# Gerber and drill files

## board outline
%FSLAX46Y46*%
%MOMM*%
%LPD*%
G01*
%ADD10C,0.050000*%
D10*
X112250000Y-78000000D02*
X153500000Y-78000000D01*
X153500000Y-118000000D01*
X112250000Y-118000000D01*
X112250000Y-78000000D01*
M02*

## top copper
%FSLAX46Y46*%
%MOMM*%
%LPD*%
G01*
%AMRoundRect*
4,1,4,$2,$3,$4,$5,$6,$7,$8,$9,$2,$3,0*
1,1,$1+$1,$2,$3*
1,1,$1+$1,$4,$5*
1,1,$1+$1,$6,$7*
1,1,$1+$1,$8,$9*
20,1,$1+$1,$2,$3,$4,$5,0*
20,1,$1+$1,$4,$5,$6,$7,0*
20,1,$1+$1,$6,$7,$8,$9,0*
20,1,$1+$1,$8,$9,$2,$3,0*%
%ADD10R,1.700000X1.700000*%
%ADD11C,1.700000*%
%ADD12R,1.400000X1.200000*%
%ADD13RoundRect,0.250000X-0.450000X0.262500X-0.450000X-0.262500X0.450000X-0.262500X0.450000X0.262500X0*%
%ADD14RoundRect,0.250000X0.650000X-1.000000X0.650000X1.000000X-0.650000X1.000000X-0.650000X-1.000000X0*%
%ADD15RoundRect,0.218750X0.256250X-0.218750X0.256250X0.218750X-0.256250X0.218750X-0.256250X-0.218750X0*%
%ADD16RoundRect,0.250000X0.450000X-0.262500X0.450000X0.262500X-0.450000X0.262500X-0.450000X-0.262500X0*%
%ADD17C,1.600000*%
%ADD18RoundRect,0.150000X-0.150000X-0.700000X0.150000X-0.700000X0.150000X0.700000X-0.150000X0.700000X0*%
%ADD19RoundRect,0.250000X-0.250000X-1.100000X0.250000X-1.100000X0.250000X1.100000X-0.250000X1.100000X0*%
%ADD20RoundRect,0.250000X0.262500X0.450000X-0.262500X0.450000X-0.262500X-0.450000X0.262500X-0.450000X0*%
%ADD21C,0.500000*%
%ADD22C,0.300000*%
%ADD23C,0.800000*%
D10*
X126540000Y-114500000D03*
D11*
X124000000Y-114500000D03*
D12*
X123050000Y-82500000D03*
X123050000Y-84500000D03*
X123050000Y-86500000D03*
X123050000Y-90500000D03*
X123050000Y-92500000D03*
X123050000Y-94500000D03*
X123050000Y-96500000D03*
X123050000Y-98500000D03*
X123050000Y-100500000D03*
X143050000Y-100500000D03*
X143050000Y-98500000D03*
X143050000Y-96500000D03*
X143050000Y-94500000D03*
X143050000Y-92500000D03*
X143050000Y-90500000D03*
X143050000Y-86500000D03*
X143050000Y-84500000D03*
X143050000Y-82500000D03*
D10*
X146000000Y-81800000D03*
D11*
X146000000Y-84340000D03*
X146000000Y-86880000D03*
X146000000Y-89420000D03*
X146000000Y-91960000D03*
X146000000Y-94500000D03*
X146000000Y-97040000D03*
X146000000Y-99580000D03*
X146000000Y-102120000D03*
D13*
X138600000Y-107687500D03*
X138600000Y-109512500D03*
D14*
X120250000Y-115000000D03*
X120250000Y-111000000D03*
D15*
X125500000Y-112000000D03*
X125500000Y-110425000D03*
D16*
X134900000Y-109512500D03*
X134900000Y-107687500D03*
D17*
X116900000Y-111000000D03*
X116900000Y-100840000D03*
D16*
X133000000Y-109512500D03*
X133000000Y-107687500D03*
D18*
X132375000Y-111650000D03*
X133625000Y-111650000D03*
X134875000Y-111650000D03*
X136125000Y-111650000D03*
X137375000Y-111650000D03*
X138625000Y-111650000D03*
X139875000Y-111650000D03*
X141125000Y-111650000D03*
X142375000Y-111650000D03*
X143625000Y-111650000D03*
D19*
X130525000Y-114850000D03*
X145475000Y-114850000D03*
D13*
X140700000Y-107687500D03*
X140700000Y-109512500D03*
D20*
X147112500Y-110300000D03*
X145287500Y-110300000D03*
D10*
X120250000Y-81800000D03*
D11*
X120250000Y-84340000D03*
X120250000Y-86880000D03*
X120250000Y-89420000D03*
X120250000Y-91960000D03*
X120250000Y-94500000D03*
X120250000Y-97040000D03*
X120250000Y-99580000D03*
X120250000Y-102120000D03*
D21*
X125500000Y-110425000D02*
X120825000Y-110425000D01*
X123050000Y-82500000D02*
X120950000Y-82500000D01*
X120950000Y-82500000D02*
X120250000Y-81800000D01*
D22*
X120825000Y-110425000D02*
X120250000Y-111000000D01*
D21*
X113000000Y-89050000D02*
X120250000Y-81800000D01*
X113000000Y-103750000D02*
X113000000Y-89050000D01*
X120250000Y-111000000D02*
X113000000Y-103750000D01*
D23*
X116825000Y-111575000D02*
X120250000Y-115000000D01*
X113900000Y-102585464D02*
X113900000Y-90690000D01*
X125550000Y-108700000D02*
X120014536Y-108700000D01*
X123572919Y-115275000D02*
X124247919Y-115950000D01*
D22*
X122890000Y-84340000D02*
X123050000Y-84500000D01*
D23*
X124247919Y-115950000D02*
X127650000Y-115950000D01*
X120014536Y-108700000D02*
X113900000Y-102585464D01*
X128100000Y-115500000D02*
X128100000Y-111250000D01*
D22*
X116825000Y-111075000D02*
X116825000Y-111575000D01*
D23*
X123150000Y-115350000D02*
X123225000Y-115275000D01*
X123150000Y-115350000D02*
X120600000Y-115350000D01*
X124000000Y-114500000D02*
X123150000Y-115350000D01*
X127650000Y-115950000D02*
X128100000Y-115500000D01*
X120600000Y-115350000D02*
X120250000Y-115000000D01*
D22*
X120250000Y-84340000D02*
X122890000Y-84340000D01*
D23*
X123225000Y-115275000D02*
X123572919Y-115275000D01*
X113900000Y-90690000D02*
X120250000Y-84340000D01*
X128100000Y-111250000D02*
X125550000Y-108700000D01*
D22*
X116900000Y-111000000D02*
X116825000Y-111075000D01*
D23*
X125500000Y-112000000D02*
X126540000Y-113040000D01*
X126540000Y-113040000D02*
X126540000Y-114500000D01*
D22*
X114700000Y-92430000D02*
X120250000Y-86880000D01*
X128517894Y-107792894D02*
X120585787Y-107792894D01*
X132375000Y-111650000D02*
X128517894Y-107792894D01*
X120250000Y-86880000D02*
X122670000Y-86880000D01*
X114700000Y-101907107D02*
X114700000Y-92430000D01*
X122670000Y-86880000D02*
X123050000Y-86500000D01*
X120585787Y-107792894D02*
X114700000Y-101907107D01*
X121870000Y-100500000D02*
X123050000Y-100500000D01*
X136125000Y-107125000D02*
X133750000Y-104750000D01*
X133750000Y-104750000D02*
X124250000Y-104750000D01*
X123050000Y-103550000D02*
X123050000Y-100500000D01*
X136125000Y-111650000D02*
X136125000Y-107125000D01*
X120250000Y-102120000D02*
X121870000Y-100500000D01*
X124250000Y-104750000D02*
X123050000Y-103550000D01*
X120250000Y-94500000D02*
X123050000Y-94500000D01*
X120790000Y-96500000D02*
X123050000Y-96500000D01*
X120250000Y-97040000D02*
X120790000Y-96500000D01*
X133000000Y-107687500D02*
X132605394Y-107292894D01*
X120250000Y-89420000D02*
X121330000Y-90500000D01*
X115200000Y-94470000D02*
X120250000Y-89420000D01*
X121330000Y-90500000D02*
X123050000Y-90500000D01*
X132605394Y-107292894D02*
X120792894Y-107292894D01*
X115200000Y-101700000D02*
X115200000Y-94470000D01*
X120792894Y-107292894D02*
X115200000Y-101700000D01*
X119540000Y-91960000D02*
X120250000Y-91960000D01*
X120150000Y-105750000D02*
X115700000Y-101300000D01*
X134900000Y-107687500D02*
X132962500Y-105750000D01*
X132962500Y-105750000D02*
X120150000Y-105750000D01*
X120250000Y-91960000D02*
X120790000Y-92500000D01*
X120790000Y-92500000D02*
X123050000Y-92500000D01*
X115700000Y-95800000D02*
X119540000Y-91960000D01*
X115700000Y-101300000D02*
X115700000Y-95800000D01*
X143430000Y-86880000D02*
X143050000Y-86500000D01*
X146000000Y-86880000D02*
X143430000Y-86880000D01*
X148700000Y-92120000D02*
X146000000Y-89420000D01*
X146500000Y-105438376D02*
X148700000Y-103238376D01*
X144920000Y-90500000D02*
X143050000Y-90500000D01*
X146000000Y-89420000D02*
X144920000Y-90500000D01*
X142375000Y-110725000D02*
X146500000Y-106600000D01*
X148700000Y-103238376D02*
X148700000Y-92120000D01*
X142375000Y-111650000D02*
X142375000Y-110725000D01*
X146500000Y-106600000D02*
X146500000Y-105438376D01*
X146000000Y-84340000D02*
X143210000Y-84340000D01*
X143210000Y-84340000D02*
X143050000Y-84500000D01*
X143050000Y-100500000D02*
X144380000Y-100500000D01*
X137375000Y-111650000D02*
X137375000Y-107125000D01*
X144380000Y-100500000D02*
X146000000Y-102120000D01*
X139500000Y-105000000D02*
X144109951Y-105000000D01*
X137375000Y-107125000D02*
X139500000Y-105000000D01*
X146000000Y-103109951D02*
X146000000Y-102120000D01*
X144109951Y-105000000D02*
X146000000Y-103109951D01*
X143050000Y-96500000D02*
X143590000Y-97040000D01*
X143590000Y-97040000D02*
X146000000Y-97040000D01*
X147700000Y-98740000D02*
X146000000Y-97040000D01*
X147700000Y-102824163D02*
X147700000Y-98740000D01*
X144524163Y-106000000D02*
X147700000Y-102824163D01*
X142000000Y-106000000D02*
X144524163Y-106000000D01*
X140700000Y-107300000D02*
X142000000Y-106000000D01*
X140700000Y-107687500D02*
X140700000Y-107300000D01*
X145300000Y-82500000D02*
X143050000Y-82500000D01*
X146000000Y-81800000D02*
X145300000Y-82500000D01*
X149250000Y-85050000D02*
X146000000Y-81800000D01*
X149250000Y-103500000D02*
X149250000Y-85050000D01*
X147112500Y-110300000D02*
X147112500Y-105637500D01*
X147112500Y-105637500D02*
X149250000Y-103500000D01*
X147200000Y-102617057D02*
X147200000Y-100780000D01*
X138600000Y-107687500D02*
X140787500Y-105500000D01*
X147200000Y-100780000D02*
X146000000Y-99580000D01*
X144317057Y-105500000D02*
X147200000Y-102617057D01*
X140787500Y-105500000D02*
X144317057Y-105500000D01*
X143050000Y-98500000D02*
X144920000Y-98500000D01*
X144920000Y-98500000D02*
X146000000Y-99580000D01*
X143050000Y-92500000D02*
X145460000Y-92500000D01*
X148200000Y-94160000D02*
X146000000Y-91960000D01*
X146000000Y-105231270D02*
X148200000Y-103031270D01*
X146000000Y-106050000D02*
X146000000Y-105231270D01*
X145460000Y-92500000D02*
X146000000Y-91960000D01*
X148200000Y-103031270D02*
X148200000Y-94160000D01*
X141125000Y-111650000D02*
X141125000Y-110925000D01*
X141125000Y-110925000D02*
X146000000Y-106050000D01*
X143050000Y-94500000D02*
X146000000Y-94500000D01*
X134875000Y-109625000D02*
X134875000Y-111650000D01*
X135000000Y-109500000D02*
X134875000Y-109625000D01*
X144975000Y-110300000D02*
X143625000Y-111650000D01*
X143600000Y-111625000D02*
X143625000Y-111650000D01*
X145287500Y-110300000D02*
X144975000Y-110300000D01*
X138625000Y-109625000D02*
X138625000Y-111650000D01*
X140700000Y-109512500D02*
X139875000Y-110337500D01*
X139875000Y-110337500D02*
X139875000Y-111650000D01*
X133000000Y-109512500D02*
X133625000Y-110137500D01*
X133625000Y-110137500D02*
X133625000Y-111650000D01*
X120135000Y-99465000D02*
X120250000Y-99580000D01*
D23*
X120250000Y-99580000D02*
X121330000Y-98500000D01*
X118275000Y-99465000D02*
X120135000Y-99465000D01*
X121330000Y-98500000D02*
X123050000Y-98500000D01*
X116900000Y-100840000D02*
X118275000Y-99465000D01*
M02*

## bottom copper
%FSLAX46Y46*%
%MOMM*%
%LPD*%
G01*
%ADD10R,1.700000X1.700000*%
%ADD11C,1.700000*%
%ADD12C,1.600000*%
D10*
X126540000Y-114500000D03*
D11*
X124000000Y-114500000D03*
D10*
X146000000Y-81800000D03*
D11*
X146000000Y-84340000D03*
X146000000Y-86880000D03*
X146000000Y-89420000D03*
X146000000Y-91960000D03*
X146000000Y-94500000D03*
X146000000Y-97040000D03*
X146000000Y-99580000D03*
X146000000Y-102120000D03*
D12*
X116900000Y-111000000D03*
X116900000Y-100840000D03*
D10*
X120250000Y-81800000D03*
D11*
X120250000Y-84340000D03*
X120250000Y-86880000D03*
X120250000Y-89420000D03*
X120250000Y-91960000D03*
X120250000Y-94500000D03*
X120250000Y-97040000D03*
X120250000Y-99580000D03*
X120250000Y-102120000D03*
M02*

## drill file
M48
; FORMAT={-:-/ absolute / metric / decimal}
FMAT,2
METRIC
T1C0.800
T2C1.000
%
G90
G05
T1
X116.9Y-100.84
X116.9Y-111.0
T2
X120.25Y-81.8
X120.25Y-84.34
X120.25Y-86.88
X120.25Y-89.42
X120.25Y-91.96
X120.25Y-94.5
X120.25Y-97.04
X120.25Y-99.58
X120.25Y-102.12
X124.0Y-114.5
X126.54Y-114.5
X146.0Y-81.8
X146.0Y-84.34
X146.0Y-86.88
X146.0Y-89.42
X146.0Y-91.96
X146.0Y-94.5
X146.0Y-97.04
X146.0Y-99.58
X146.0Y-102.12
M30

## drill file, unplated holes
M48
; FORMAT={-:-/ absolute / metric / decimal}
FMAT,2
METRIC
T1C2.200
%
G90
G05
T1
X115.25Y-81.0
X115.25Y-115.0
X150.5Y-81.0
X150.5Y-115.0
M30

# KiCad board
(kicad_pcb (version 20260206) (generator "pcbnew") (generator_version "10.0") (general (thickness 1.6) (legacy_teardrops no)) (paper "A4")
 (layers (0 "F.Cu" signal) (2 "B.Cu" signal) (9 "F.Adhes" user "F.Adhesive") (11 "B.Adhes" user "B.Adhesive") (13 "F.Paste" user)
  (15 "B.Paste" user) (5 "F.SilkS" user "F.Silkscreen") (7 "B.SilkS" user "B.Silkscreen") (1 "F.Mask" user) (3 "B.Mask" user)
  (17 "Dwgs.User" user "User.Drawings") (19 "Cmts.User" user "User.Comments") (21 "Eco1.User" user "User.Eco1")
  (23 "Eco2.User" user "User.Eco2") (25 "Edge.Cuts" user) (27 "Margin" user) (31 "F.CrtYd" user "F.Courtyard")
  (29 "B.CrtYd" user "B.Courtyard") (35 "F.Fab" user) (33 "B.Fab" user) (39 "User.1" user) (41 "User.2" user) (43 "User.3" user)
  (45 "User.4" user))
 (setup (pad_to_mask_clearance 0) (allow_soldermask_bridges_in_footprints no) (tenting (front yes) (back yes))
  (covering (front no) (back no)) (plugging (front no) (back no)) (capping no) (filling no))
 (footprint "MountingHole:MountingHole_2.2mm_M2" (layer "F.Cu") (at 115.25 81)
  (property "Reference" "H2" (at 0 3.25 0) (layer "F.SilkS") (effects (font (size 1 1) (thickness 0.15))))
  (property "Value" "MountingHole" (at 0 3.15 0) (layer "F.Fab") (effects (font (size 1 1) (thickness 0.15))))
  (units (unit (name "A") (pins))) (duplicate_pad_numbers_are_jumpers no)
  (pad "" np_thru_hole circle (at 0 0) (size 2.2 2.2) (drill 2.2) (layers "*.Cu" "*.Mask")))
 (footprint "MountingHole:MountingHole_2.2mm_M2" (layer "F.Cu") (at 115.25 115)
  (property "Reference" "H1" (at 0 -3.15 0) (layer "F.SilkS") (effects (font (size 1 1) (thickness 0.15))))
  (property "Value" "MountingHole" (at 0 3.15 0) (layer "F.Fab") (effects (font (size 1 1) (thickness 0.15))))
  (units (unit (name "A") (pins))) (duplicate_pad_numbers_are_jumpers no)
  (pad "" np_thru_hole circle (at 0 0) (size 2.2 2.2) (drill 2.2) (layers "*.Cu" "*.Mask")))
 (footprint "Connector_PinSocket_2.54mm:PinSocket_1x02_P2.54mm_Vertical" (layer "F.Cu") (at 126.54 114.5 -90)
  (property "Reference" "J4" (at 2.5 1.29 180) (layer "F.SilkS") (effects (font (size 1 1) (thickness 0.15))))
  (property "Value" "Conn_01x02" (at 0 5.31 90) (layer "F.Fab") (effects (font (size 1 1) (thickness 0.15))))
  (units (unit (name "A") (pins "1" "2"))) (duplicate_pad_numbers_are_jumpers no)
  (pad "1" thru_hole rect (at 0 0 270) (size 1.7 1.7) (drill 1) (layers "*.Cu" "*.Mask") (remove_unused_layers no) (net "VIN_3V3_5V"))
  (pad "2" thru_hole circle (at 0 2.54 270) (size 1.7 1.7) (drill 1) (layers "*.Cu" "*.Mask") (remove_unused_layers no) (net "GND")))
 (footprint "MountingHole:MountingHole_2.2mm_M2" (layer "F.Cu") (at 150.5 115)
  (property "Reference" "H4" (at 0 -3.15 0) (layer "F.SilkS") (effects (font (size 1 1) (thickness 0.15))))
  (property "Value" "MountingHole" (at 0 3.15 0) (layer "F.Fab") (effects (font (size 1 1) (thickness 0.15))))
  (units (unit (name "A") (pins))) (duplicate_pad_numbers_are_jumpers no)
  (pad "" np_thru_hole circle (at 0 0) (size 2.2 2.2) (drill 2.2) (layers "*.Cu" "*.Mask")))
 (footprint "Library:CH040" (layer "F.Cu") (at 133.05 91.5)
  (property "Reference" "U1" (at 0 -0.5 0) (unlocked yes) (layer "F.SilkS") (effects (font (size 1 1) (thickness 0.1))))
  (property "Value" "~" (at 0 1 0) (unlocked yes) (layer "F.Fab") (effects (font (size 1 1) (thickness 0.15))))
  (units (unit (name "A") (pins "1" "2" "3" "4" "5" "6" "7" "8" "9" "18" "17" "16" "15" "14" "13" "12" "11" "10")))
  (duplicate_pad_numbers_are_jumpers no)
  (pad "1" smd rect (at -10 -9) (size 1.4 1.2) (layers "F.Cu" "F.Mask" "F.Paste") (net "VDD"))
  (pad "2" smd rect (at -10 -7) (size 1.4 1.2) (layers "F.Cu" "F.Mask" "F.Paste") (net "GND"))
  (pad "3" smd rect (at -10 -5) (size 1.4 1.2) (layers "F.Cu" "F.Mask" "F.Paste") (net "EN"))
  (pad "4" smd rect (at -10 -1) (size 1.4 1.2) (layers "F.Cu" "F.Mask" "F.Paste") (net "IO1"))
  (pad "5" smd rect (at -10 1) (size 1.4 1.2) (layers "F.Cu" "F.Mask" "F.Paste") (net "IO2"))
  (pad "6" smd rect (at -10 3) (size 1.4 1.2) (layers "F.Cu" "F.Mask" "F.Paste") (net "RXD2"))
  (pad "7" smd rect (at -10 5) (size 1.4 1.2) (layers "F.Cu" "F.Mask" "F.Paste") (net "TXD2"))
  (pad "8" smd rect (at -10 7) (size 1.4 1.2) (layers "F.Cu" "F.Mask" "F.Paste") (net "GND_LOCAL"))
  (pad "9" smd rect (at -10 9) (size 1.4 1.2) (layers "F.Cu" "F.Mask" "F.Paste") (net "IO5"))
  (pad "10" smd rect (at 10 9) (size 1.4 1.2) (layers "F.Cu" "F.Mask" "F.Paste") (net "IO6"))
  (pad "11" smd rect (at 10 7) (size 1.4 1.2) (layers "F.Cu" "F.Mask" "F.Paste") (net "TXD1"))
  (pad "12" smd rect (at 10 5) (size 1.4 1.2) (layers "F.Cu" "F.Mask" "F.Paste") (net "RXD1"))
  (pad "13" smd rect (at 10 3) (size 1.4 1.2) (layers "F.Cu" "F.Mask" "F.Paste") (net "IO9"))
  (pad "14" smd rect (at 10 1) (size 1.4 1.2) (layers "F.Cu" "F.Mask" "F.Paste") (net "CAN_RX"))
  (pad "15" smd rect (at 10 -1) (size 1.4 1.2) (layers "F.Cu" "F.Mask" "F.Paste") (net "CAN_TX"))
  (pad "16" smd rect (at 10 -5) (size 1.4 1.2) (layers "F.Cu" "F.Mask" "F.Paste") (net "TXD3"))
  (pad "17" smd rect (at 10 -7) (size 1.4 1.2) (layers "F.Cu" "F.Mask" "F.Paste") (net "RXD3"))
  (pad "18" smd rect (at 10 -9) (size 1.4 1.2) (layers "F.Cu" "F.Mask" "F.Paste") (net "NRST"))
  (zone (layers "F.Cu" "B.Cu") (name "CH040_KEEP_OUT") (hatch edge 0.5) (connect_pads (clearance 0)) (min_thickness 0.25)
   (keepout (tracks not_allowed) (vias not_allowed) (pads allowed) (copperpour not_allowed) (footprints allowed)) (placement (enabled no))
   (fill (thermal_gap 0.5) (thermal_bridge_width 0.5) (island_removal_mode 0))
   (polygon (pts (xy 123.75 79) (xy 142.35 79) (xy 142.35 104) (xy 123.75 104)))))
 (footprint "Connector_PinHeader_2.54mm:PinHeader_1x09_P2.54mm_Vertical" (layer "F.Cu") (at 146 81.8)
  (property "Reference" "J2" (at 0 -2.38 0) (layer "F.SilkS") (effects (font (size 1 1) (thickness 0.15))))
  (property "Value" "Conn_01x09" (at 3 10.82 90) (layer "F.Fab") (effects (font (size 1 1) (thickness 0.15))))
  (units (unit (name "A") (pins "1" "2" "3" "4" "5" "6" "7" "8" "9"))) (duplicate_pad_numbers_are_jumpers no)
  (pad "1" thru_hole rect (at 0 0) (size 1.7 1.7) (drill 1) (layers "*.Cu" "*.Mask") (remove_unused_layers no) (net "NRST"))
  (pad "2" thru_hole circle (at 0 2.54) (size 1.7 1.7) (drill 1) (layers "*.Cu" "*.Mask") (remove_unused_layers no) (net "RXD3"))
  (pad "3" thru_hole circle (at 0 5.08) (size 1.7 1.7) (drill 1) (layers "*.Cu" "*.Mask") (remove_unused_layers no) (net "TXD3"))
  (pad "4" thru_hole circle (at 0 7.62) (size 1.7 1.7) (drill 1) (layers "*.Cu" "*.Mask") (remove_unused_layers no) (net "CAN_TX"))
  (pad "5" thru_hole circle (at 0 10.16) (size 1.7 1.7) (drill 1) (layers "*.Cu" "*.Mask") (remove_unused_layers no) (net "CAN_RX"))
  (pad "6" thru_hole circle (at 0 12.7) (size 1.7 1.7) (drill 1) (layers "*.Cu" "*.Mask") (remove_unused_layers no) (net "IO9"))
  (pad "7" thru_hole circle (at 0 15.24) (size 1.7 1.7) (drill 1) (layers "*.Cu" "*.Mask") (remove_unused_layers no) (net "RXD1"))
  (pad "8" thru_hole circle (at 0 17.78) (size 1.7 1.7) (drill 1) (layers "*.Cu" "*.Mask") (remove_unused_layers no) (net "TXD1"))
  (pad "9" thru_hole circle (at 0 20.32) (size 1.7 1.7) (drill 1) (layers "*.Cu" "*.Mask") (remove_unused_layers no) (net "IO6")))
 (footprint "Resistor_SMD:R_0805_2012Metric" (layer "F.Cu") (at 138.6 108.6 -90)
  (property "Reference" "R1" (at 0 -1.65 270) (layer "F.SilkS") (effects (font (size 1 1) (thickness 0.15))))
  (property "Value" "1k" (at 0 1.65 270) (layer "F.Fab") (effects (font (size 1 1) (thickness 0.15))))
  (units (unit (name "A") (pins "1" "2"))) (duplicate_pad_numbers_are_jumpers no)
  (pad "1" smd roundrect (at -0.9125 0 270) (size 1.025 1.4) (layers "F.Cu" "F.Mask" "F.Paste") (roundrect_rratio 0.243902) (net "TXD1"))
  (pad "2" smd roundrect (at 0.9125 0 270) (size 1.025 1.4) (layers "F.Cu" "F.Mask" "F.Paste") (roundrect_rratio 0.243902) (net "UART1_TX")))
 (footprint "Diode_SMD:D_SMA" (layer "F.Cu") (at 120.25 113 90)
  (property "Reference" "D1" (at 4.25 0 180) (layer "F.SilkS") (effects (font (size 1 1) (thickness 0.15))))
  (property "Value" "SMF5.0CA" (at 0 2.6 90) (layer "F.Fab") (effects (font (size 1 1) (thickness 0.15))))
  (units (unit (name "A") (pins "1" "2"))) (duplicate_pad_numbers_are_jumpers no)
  (pad "1" smd roundrect (at -2 0 90) (size 2.5 1.8) (layers "F.Cu" "F.Mask" "F.Paste") (roundrect_rratio 0.1388888889) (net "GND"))
  (pad "2" smd roundrect (at 2 0 90) (size 2.5 1.8) (layers "F.Cu" "F.Mask" "F.Paste") (roundrect_rratio 0.1388888889) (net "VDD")))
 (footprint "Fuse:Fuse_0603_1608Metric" (layer "F.Cu") (at 125.5 111.2125 90)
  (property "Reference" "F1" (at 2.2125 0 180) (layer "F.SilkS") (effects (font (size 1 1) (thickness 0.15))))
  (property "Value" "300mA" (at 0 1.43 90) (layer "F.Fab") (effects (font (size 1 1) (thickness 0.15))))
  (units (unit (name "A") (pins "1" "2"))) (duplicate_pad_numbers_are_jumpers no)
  (pad "1" smd roundrect (at -0.7875 0 90) (size 0.875 0.95) (layers "F.Cu" "F.Mask" "F.Paste") (roundrect_rratio 0.25) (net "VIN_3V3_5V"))
  (pad "2" smd roundrect (at 0.7875 0 90) (size 0.875 0.95) (layers "F.Cu" "F.Mask" "F.Paste") (roundrect_rratio 0.25) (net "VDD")))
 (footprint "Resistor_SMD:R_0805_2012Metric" (layer "F.Cu") (at 134.9 108.6 90)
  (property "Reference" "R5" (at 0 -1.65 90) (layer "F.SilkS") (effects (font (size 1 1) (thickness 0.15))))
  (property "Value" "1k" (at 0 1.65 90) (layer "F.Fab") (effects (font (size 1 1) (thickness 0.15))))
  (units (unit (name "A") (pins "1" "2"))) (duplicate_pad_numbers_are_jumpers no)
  (pad "1" smd roundrect (at -0.9125 0 90) (size 1.025 1.4) (layers "F.Cu" "F.Mask" "F.Paste") (roundrect_rratio 0.243902) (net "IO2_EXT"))
  (pad "2" smd roundrect (at 0.9125 0 90) (size 1.025 1.4) (layers "F.Cu" "F.Mask" "F.Paste") (roundrect_rratio 0.243902) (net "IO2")))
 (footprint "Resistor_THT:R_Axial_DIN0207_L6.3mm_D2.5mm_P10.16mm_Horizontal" (layer "F.Cu") (at 116.9 111 90)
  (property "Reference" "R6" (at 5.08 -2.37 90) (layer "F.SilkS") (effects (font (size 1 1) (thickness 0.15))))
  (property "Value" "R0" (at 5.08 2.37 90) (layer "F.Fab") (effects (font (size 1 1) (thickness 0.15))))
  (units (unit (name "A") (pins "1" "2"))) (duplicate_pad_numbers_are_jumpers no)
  (pad "1" thru_hole circle (at 0 0 90) (size 1.6 1.6) (drill 0.8) (layers "*.Cu" "*.Mask") (remove_unused_layers no) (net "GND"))
  (pad "2" thru_hole circle (at 10.16 0 90) (size 1.6 1.6) (drill 0.8) (layers "*.Cu" "*.Mask") (remove_unused_layers no) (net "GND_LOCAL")))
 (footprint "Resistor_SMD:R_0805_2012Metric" (layer "F.Cu") (at 133 108.6 90)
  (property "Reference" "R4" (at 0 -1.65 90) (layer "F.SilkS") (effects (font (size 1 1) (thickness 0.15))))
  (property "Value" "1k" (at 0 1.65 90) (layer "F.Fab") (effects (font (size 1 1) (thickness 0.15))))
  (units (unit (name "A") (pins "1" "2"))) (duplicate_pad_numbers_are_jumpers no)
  (pad "1" smd roundrect (at -0.9125 0 90) (size 1.025 1.4) (layers "F.Cu" "F.Mask" "F.Paste") (roundrect_rratio 0.243902) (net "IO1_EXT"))
  (pad "2" smd roundrect (at 0.9125 0 90) (size 1.025 1.4) (layers "F.Cu" "F.Mask" "F.Paste") (roundrect_rratio 0.243902) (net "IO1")))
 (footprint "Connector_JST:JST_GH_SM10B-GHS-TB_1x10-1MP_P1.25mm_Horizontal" (layer "F.Cu") (at 138 113.5)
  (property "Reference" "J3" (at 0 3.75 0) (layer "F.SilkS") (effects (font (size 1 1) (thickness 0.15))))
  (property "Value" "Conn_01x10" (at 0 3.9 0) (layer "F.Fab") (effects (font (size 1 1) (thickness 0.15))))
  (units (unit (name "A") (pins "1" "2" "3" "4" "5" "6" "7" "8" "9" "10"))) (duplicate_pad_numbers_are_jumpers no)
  (pad "1" smd roundrect (at -5.625 -1.85) (size 0.6 1.7) (layers "F.Cu" "F.Mask" "F.Paste") (roundrect_rratio 0.25) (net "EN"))
  (pad "2" smd roundrect (at -4.375 -1.85) (size 0.6 1.7) (layers "F.Cu" "F.Mask" "F.Paste") (roundrect_rratio 0.25) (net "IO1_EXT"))
  (pad "3" smd roundrect (at -3.125 -1.85) (size 0.6 1.7) (layers "F.Cu" "F.Mask" "F.Paste") (roundrect_rratio 0.25) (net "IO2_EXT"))
  (pad "4" smd roundrect (at -1.875 -1.85) (size 0.6 1.7) (layers "F.Cu" "F.Mask" "F.Paste") (roundrect_rratio 0.25) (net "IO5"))
  (pad "5" smd roundrect (at -0.625 -1.85) (size 0.6 1.7) (layers "F.Cu" "F.Mask" "F.Paste") (roundrect_rratio 0.25) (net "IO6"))
  (pad "6" smd roundrect (at 0.625 -1.85) (size 0.6 1.7) (layers "F.Cu" "F.Mask" "F.Paste") (roundrect_rratio 0.25) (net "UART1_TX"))
  (pad "7" smd roundrect (at 1.875 -1.85) (size 0.6 1.7) (layers "F.Cu" "F.Mask" "F.Paste") (roundrect_rratio 0.25) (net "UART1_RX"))
  (pad "8" smd roundrect (at 3.125 -1.85) (size 0.6 1.7) (layers "F.Cu" "F.Mask" "F.Paste") (roundrect_rratio 0.25) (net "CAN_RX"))
  (pad "9" smd roundrect (at 4.375 -1.85) (size 0.6 1.7) (layers "F.Cu" "F.Mask" "F.Paste") (roundrect_rratio 0.25) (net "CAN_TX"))
  (pad "10" smd roundrect (at 5.625 -1.85) (size 0.6 1.7) (layers "F.Cu" "F.Mask" "F.Paste") (roundrect_rratio 0.25) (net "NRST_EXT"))
  (pad "MP" smd roundrect (at -7.475 1.35) (size 1 2.7) (layers "F.Cu" "F.Mask" "F.Paste") (roundrect_rratio 0.25))
  (pad "MP" smd roundrect (at 7.475 1.35) (size 1 2.7) (layers "F.Cu" "F.Mask" "F.Paste") (roundrect_rratio 0.25)))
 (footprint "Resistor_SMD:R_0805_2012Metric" (layer "F.Cu") (at 140.7 108.6 -90)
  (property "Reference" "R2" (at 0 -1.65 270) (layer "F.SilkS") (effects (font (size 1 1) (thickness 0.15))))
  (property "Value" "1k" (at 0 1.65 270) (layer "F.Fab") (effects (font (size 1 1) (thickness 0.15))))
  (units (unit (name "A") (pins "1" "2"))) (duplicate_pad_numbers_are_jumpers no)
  (pad "1" smd roundrect (at -0.9125 0 270) (size 1.025 1.4) (layers "F.Cu" "F.Mask" "F.Paste") (roundrect_rratio 0.243902) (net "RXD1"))
  (pad "2" smd roundrect (at 0.9125 0 270) (size 1.025 1.4) (layers "F.Cu" "F.Mask" "F.Paste") (roundrect_rratio 0.243902) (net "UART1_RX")))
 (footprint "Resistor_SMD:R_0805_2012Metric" (layer "F.Cu") (at 146.2 110.3 180)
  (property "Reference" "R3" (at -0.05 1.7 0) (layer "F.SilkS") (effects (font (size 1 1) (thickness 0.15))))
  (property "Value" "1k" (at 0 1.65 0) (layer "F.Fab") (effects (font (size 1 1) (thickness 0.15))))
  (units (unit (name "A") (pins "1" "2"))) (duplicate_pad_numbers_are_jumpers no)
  (pad "1" smd roundrect (at -0.9125 0 180) (size 1.025 1.4) (layers "F.Cu" "F.Mask" "F.Paste") (roundrect_rratio 0.243902) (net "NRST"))
  (pad "2" smd roundrect (at 0.9125 0 180) (size 1.025 1.4) (layers "F.Cu" "F.Mask" "F.Paste") (roundrect_rratio 0.243902) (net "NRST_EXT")))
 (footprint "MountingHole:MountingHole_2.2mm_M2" (layer "F.Cu") (at 150.5 81)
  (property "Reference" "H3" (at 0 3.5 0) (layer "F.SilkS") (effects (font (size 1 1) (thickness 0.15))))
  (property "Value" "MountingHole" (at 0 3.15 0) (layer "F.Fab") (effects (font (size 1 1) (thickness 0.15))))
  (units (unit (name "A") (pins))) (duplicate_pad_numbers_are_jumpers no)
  (pad "" np_thru_hole circle (at 0 0) (size 2.2 2.2) (drill 2.2) (layers "*.Cu" "*.Mask")))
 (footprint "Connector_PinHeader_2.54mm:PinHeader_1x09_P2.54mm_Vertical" (layer "F.Cu") (at 120.25 81.8)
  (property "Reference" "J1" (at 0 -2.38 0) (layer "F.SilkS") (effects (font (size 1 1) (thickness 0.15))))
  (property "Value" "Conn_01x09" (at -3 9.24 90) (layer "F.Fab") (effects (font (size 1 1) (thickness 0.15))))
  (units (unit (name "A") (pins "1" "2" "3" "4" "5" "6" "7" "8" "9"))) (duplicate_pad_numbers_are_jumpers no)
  (pad "1" thru_hole rect (at 0 0) (size 1.7 1.7) (drill 1) (layers "*.Cu" "*.Mask") (remove_unused_layers no) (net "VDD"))
  (pad "2" thru_hole circle (at 0 2.54) (size 1.7 1.7) (drill 1) (layers "*.Cu" "*.Mask") (remove_unused_layers no) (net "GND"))
  (pad "3" thru_hole circle (at 0 5.08) (size 1.7 1.7) (drill 1) (layers "*.Cu" "*.Mask") (remove_unused_layers no) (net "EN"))
  (pad "4" thru_hole circle (at 0 7.62) (size 1.7 1.7) (drill 1) (layers "*.Cu" "*.Mask") (remove_unused_layers no) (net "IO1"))
  (pad "5" thru_hole circle (at 0 10.16) (size 1.7 1.7) (drill 1) (layers "*.Cu" "*.Mask") (remove_unused_layers no) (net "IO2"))
  (pad "6" thru_hole circle (at 0 12.7) (size 1.7 1.7) (drill 1) (layers "*.Cu" "*.Mask") (remove_unused_layers no) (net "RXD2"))
  (pad "7" thru_hole circle (at 0 15.24) (size 1.7 1.7) (drill 1) (layers "*.Cu" "*.Mask") (remove_unused_layers no) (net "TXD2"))
  (pad "8" thru_hole circle (at 0 17.78) (size 1.7 1.7) (drill 1) (layers "*.Cu" "*.Mask") (remove_unused_layers no) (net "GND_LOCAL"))
  (pad "9" thru_hole circle (at 0 20.32) (size 1.7 1.7) (drill 1) (layers "*.Cu" "*.Mask") (remove_unused_layers no) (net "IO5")))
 (gr_rect (start 112.25 78) (end 153.5 118) (stroke (width 0.05) (type default)) (fill no) (layer "Edge.Cuts"))
 (segment (start 125.5 112) (end 126.54 113.04) (width 0.8) (layer "F.Cu") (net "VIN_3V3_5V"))
 (segment (start 126.54 113.04) (end 126.54 114.5) (width 0.8) (layer "F.Cu") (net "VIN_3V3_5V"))
 (segment (start 116.825 111.575) (end 120.25 115) (width 0.8) (layer "F.Cu") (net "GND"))
 (segment (start 113.9 102.585464) (end 113.9 90.69) (width 0.8) (layer "F.Cu") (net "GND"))
 (segment (start 125.55 108.7) (end 120.014536 108.7) (width 0.8) (layer "F.Cu") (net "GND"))
 (segment (start 123.572919 115.275) (end 124.247919 115.95) (width 0.8) (layer "F.Cu") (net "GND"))
 (segment (start 122.89 84.34) (end 123.05 84.5) (width 0.3) (layer "F.Cu") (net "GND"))
 (segment (start 124.247919 115.95) (end 127.65 115.95) (width 0.8) (layer "F.Cu") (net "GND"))
 (segment (start 120.014536 108.7) (end 113.9 102.585464) (width 0.8) (layer "F.Cu") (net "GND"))
 (segment (start 128.1 115.5) (end 128.1 111.25) (width 0.8) (layer "F.Cu") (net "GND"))
 (segment (start 116.825 111.075) (end 116.825 111.575) (width 0.3) (layer "F.Cu") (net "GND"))
 (segment (start 123.15 115.35) (end 123.225 115.275) (width 0.8) (layer "F.Cu") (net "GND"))
 (segment (start 123.15 115.35) (end 120.6 115.35) (width 0.8) (layer "F.Cu") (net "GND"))
 (segment (start 124 114.5) (end 123.15 115.35) (width 0.8) (layer "F.Cu") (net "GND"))
 (segment (start 127.65 115.95) (end 128.1 115.5) (width 0.8) (layer "F.Cu") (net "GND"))
 (segment (start 120.6 115.35) (end 120.25 115) (width 0.8) (layer "F.Cu") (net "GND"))
 (segment (start 120.25 84.34) (end 122.89 84.34) (width 0.3) (layer "F.Cu") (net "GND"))
 (segment (start 123.225 115.275) (end 123.572919 115.275) (width 0.8) (layer "F.Cu") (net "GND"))
 (segment (start 113.9 90.69) (end 120.25 84.34) (width 0.8) (layer "F.Cu") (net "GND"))
 (segment (start 128.1 111.25) (end 125.55 108.7) (width 0.8) (layer "F.Cu") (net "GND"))
 (segment (start 116.9 111) (end 116.825 111.075) (width 0.3) (layer "F.Cu") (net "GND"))
 (segment (start 125.5 110.425) (end 120.825 110.425) (width 0.5) (layer "F.Cu") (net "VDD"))
 (segment (start 123.05 82.5) (end 120.95 82.5) (width 0.5) (layer "F.Cu") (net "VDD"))
 (segment (start 120.95 82.5) (end 120.25 81.8) (width 0.5) (layer "F.Cu") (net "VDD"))
 (segment (start 120.825 110.425) (end 120.25 111) (width 0.3) (layer "F.Cu") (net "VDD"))
 (segment (start 113 89.05) (end 120.25 81.8) (width 0.5) (layer "F.Cu") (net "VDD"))
 (segment (start 113 103.75) (end 113 89.05) (width 0.5) (layer "F.Cu") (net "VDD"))
 (segment (start 120.25 111) (end 113 103.75) (width 0.5) (layer "F.Cu") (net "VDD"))
 (segment (start 114.7 92.43) (end 120.25 86.88) (width 0.3) (layer "F.Cu") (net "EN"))
 (segment (start 128.517894 107.792894) (end 120.585787 107.792894) (width 0.3) (layer "F.Cu") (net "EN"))
 (segment (start 132.375 111.65) (end 128.517894 107.792894) (width 0.3) (layer "F.Cu") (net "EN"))
 (segment (start 120.25 86.88) (end 122.67 86.88) (width 0.3) (layer "F.Cu") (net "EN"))
 (segment (start 114.7 101.907107) (end 114.7 92.43) (width 0.3) (layer "F.Cu") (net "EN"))
 (segment (start 122.67 86.88) (end 123.05 86.5) (width 0.3) (layer "F.Cu") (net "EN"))
 (segment (start 120.585787 107.792894) (end 114.7 101.907107) (width 0.3) (layer "F.Cu") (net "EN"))
 (segment (start 133 107.6875) (end 132.605394 107.292894) (width 0.3) (layer "F.Cu") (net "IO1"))
 (segment (start 120.25 89.42) (end 121.33 90.5) (width 0.3) (layer "F.Cu") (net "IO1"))
 (segment (start 115.2 94.47) (end 120.25 89.42) (width 0.3) (layer "F.Cu") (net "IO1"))
 (segment (start 121.33 90.5) (end 123.05 90.5) (width 0.3) (layer "F.Cu") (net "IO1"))
 (segment (start 132.605394 107.292894) (end 120.792894 107.292894) (width 0.3) (layer "F.Cu") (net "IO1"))
 (segment (start 115.2 101.7) (end 115.2 94.47) (width 0.3) (layer "F.Cu") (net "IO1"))
 (segment (start 120.792894 107.292894) (end 115.2 101.7) (width 0.3) (layer "F.Cu") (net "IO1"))
 (segment (start 119.54 91.96) (end 120.25 91.96) (width 0.3) (layer "F.Cu") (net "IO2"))
 (segment (start 120.15 105.75) (end 115.7 101.3) (width 0.3) (layer "F.Cu") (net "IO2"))
 (segment (start 134.9 107.6875) (end 132.9625 105.75) (width 0.3) (layer "F.Cu") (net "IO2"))
 (segment (start 132.9625 105.75) (end 120.15 105.75) (width 0.3) (layer "F.Cu") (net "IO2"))
 (segment (start 120.25 91.96) (end 120.79 92.5) (width 0.3) (layer "F.Cu") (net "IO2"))
 (segment (start 120.79 92.5) (end 123.05 92.5) (width 0.3) (layer "F.Cu") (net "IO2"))
 (segment (start 115.7 95.8) (end 119.54 91.96) (width 0.3) (layer "F.Cu") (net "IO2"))
 (segment (start 115.7 101.3) (end 115.7 95.8) (width 0.3) (layer "F.Cu") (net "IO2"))
 (segment (start 120.25 94.5) (end 123.05 94.5) (width 0.3) (layer "F.Cu") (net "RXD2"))
 (segment (start 120.79 96.5) (end 123.05 96.5) (width 0.3) (layer "F.Cu") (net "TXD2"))
 (segment (start 120.25 97.04) (end 120.79 96.5) (width 0.3) (layer "F.Cu") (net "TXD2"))
 (segment (start 120.135 99.465) (end 120.25 99.58) (width 0.3) (layer "F.Cu") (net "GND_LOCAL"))
 (segment (start 120.25 99.58) (end 121.33 98.5) (width 0.8) (layer "F.Cu") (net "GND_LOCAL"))
 (segment (start 118.275 99.465) (end 120.135 99.465) (width 0.8) (layer "F.Cu") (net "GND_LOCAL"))
 (segment (start 121.33 98.5) (end 123.05 98.5) (width 0.8) (layer "F.Cu") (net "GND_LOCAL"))
 (segment (start 116.9 100.84) (end 118.275 99.465) (width 0.8) (layer "F.Cu") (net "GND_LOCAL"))
 (segment (start 121.87 100.5) (end 123.05 100.5) (width 0.3) (layer "F.Cu") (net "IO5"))
 (segment (start 136.125 107.125) (end 133.75 104.75) (width 0.3) (layer "F.Cu") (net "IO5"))
 (segment (start 133.75 104.75) (end 124.25 104.75) (width 0.3) (layer "F.Cu") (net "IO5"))
 (segment (start 123.05 103.55) (end 123.05 100.5) (width 0.3) (layer "F.Cu") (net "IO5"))
 (segment (start 136.125 111.65) (end 136.125 107.125) (width 0.3) (layer "F.Cu") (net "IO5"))
 (segment (start 120.25 102.12) (end 121.87 100.5) (width 0.3) (layer "F.Cu") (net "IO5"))
 (segment (start 124.25 104.75) (end 123.05 103.55) (width 0.3) (layer "F.Cu") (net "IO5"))
 (segment (start 143.05 100.5) (end 144.38 100.5) (width 0.3) (layer "F.Cu") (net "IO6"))
 (segment (start 137.375 111.65) (end 137.375 107.125) (width 0.3) (layer "F.Cu") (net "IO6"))
 (segment (start 144.38 100.5) (end 146 102.12) (width 0.3) (layer "F.Cu") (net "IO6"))
 (segment (start 139.5 105) (end 144.109951 105) (width 0.3) (layer "F.Cu") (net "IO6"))
 (segment (start 137.375 107.125) (end 139.5 105) (width 0.3) (layer "F.Cu") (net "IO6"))
 (segment (start 146 103.109951) (end 146 102.12) (width 0.3) (layer "F.Cu") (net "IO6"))
 (segment (start 144.109951 105) (end 146 103.109951) (width 0.3) (layer "F.Cu") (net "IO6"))
 (segment (start 147.2 102.617057) (end 147.2 100.78) (width 0.3) (layer "F.Cu") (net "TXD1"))
 (segment (start 138.6 107.6875) (end 140.7875 105.5) (width 0.3) (layer "F.Cu") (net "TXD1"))
 (segment (start 147.2 100.78) (end 146 99.58) (width 0.3) (layer "F.Cu") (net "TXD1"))
 (segment (start 144.317057 105.5) (end 147.2 102.617057) (width 0.3) (layer "F.Cu") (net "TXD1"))
 (segment (start 140.7875 105.5) (end 144.317057 105.5) (width 0.3) (layer "F.Cu") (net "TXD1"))
 (segment (start 143.05 98.5) (end 144.92 98.5) (width 0.3) (layer "F.Cu") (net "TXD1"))
 (segment (start 144.92 98.5) (end 146 99.58) (width 0.3) (layer "F.Cu") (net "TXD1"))
 (segment (start 143.05 96.5) (end 143.59 97.04) (width 0.3) (layer "F.Cu") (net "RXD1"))
 (segment (start 143.59 97.04) (end 146 97.04) (width 0.3) (layer "F.Cu") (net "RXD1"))
 (segment (start 147.7 98.74) (end 146 97.04) (width 0.3) (layer "F.Cu") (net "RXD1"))
 (segment (start 147.7 102.824163) (end 147.7 98.74) (width 0.3) (layer "F.Cu") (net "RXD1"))
 (segment (start 144.524163 106) (end 147.7 102.824163) (width 0.3) (layer "F.Cu") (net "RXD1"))
 (segment (start 142 106) (end 144.524163 106) (width 0.3) (layer "F.Cu") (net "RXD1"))
 (segment (start 140.7 107.3) (end 142 106) (width 0.3) (layer "F.Cu") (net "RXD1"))
 (segment (start 140.7 107.6875) (end 140.7 107.3) (width 0.3) (layer "F.Cu") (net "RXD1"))
 (segment (start 143.05 94.5) (end 146 94.5) (width 0.3) (layer "F.Cu") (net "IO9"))
 (segment (start 143.05 92.5) (end 145.46 92.5) (width 0.3) (layer "F.Cu") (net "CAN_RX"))
 (segment (start 148.2 94.16) (end 146 91.96) (width 0.3) (layer "F.Cu") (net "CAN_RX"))
 (segment (start 146 105.23127) (end 148.2 103.03127) (width 0.3) (layer "F.Cu") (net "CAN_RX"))
 (segment (start 146 106.05) (end 146 105.23127) (width 0.3) (layer "F.Cu") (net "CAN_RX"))
 (segment (start 145.46 92.5) (end 146 91.96) (width 0.3) (layer "F.Cu") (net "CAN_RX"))
 (segment (start 148.2 103.03127) (end 148.2 94.16) (width 0.3) (layer "F.Cu") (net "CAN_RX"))
 (segment (start 141.125 111.65) (end 141.125 110.925) (width 0.3) (layer "F.Cu") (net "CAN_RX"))
 (segment (start 141.125 110.925) (end 146 106.05) (width 0.3) (layer "F.Cu") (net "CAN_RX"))
 (segment (start 148.7 92.12) (end 146 89.42) (width 0.3) (layer "F.Cu") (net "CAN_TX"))
 (segment (start 146.5 105.438376) (end 148.7 103.238376) (width 0.3) (layer "F.Cu") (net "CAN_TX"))
 (segment (start 144.92 90.5) (end 143.05 90.5) (width 0.3) (layer "F.Cu") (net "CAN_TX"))
 (segment (start 146 89.42) (end 144.92 90.5) (width 0.3) (layer "F.Cu") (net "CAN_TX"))
 (segment (start 142.375 110.725) (end 146.5 106.6) (width 0.3) (layer "F.Cu") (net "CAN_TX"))
 (segment (start 148.7 103.238376) (end 148.7 92.12) (width 0.3) (layer "F.Cu") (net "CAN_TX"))
 (segment (start 142.375 111.65) (end 142.375 110.725) (width 0.3) (layer "F.Cu") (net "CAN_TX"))
 (segment (start 146.5 106.6) (end 146.5 105.438376) (width 0.3) (layer "F.Cu") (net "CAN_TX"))
 (segment (start 143.43 86.88) (end 143.05 86.5) (width 0.3) (layer "F.Cu") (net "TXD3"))
 (segment (start 146 86.88) (end 143.43 86.88) (width 0.3) (layer "F.Cu") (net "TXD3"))
 (segment (start 146 84.34) (end 143.21 84.34) (width 0.3) (layer "F.Cu") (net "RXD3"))
 (segment (start 143.21 84.34) (end 143.05 84.5) (width 0.3) (layer "F.Cu") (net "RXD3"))
 (segment (start 145.3 82.5) (end 143.05 82.5) (width 0.3) (layer "F.Cu") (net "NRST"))
 (segment (start 146 81.8) (end 145.3 82.5) (width 0.3) (layer "F.Cu") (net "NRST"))
 (segment (start 149.25 85.05) (end 146 81.8) (width 0.3) (layer "F.Cu") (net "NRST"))
 (segment (start 149.25 103.5) (end 149.25 85.05) (width 0.3) (layer "F.Cu") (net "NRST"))
 (segment (start 147.1125 110.3) (end 147.1125 105.6375) (width 0.3) (layer "F.Cu") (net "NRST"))
 (segment (start 147.1125 105.6375) (end 149.25 103.5) (width 0.3) (layer "F.Cu") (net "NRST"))
 (segment (start 138.625 109.625) (end 138.625 111.65) (width 0.3) (layer "F.Cu") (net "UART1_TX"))
 (segment (start 134.875 109.625) (end 134.875 111.65) (width 0.3) (layer "F.Cu") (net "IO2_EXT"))
 (segment (start 135 109.5) (end 134.875 109.625) (width 0.3) (layer "F.Cu") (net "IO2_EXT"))
 (segment (start 133 109.5125) (end 133.625 110.1375) (width 0.3) (layer "F.Cu") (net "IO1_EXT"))
 (segment (start 133.625 110.1375) (end 133.625 111.65) (width 0.3) (layer "F.Cu") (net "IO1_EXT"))
 (segment (start 140.7 109.5125) (end 139.875 110.3375) (width 0.3) (layer "F.Cu") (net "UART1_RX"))
 (segment (start 139.875 110.3375) (end 139.875 111.65) (width 0.3) (layer "F.Cu") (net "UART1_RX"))
 (segment (start 144.975 110.3) (end 143.625 111.65) (width 0.3) (layer "F.Cu") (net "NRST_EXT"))
 (segment (start 143.6 111.625) (end 143.625 111.65) (width 0.3) (layer "F.Cu") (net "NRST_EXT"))
 (segment (start 145.2875 110.3) (end 144.975 110.3) (width 0.3) (layer "F.Cu") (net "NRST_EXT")))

